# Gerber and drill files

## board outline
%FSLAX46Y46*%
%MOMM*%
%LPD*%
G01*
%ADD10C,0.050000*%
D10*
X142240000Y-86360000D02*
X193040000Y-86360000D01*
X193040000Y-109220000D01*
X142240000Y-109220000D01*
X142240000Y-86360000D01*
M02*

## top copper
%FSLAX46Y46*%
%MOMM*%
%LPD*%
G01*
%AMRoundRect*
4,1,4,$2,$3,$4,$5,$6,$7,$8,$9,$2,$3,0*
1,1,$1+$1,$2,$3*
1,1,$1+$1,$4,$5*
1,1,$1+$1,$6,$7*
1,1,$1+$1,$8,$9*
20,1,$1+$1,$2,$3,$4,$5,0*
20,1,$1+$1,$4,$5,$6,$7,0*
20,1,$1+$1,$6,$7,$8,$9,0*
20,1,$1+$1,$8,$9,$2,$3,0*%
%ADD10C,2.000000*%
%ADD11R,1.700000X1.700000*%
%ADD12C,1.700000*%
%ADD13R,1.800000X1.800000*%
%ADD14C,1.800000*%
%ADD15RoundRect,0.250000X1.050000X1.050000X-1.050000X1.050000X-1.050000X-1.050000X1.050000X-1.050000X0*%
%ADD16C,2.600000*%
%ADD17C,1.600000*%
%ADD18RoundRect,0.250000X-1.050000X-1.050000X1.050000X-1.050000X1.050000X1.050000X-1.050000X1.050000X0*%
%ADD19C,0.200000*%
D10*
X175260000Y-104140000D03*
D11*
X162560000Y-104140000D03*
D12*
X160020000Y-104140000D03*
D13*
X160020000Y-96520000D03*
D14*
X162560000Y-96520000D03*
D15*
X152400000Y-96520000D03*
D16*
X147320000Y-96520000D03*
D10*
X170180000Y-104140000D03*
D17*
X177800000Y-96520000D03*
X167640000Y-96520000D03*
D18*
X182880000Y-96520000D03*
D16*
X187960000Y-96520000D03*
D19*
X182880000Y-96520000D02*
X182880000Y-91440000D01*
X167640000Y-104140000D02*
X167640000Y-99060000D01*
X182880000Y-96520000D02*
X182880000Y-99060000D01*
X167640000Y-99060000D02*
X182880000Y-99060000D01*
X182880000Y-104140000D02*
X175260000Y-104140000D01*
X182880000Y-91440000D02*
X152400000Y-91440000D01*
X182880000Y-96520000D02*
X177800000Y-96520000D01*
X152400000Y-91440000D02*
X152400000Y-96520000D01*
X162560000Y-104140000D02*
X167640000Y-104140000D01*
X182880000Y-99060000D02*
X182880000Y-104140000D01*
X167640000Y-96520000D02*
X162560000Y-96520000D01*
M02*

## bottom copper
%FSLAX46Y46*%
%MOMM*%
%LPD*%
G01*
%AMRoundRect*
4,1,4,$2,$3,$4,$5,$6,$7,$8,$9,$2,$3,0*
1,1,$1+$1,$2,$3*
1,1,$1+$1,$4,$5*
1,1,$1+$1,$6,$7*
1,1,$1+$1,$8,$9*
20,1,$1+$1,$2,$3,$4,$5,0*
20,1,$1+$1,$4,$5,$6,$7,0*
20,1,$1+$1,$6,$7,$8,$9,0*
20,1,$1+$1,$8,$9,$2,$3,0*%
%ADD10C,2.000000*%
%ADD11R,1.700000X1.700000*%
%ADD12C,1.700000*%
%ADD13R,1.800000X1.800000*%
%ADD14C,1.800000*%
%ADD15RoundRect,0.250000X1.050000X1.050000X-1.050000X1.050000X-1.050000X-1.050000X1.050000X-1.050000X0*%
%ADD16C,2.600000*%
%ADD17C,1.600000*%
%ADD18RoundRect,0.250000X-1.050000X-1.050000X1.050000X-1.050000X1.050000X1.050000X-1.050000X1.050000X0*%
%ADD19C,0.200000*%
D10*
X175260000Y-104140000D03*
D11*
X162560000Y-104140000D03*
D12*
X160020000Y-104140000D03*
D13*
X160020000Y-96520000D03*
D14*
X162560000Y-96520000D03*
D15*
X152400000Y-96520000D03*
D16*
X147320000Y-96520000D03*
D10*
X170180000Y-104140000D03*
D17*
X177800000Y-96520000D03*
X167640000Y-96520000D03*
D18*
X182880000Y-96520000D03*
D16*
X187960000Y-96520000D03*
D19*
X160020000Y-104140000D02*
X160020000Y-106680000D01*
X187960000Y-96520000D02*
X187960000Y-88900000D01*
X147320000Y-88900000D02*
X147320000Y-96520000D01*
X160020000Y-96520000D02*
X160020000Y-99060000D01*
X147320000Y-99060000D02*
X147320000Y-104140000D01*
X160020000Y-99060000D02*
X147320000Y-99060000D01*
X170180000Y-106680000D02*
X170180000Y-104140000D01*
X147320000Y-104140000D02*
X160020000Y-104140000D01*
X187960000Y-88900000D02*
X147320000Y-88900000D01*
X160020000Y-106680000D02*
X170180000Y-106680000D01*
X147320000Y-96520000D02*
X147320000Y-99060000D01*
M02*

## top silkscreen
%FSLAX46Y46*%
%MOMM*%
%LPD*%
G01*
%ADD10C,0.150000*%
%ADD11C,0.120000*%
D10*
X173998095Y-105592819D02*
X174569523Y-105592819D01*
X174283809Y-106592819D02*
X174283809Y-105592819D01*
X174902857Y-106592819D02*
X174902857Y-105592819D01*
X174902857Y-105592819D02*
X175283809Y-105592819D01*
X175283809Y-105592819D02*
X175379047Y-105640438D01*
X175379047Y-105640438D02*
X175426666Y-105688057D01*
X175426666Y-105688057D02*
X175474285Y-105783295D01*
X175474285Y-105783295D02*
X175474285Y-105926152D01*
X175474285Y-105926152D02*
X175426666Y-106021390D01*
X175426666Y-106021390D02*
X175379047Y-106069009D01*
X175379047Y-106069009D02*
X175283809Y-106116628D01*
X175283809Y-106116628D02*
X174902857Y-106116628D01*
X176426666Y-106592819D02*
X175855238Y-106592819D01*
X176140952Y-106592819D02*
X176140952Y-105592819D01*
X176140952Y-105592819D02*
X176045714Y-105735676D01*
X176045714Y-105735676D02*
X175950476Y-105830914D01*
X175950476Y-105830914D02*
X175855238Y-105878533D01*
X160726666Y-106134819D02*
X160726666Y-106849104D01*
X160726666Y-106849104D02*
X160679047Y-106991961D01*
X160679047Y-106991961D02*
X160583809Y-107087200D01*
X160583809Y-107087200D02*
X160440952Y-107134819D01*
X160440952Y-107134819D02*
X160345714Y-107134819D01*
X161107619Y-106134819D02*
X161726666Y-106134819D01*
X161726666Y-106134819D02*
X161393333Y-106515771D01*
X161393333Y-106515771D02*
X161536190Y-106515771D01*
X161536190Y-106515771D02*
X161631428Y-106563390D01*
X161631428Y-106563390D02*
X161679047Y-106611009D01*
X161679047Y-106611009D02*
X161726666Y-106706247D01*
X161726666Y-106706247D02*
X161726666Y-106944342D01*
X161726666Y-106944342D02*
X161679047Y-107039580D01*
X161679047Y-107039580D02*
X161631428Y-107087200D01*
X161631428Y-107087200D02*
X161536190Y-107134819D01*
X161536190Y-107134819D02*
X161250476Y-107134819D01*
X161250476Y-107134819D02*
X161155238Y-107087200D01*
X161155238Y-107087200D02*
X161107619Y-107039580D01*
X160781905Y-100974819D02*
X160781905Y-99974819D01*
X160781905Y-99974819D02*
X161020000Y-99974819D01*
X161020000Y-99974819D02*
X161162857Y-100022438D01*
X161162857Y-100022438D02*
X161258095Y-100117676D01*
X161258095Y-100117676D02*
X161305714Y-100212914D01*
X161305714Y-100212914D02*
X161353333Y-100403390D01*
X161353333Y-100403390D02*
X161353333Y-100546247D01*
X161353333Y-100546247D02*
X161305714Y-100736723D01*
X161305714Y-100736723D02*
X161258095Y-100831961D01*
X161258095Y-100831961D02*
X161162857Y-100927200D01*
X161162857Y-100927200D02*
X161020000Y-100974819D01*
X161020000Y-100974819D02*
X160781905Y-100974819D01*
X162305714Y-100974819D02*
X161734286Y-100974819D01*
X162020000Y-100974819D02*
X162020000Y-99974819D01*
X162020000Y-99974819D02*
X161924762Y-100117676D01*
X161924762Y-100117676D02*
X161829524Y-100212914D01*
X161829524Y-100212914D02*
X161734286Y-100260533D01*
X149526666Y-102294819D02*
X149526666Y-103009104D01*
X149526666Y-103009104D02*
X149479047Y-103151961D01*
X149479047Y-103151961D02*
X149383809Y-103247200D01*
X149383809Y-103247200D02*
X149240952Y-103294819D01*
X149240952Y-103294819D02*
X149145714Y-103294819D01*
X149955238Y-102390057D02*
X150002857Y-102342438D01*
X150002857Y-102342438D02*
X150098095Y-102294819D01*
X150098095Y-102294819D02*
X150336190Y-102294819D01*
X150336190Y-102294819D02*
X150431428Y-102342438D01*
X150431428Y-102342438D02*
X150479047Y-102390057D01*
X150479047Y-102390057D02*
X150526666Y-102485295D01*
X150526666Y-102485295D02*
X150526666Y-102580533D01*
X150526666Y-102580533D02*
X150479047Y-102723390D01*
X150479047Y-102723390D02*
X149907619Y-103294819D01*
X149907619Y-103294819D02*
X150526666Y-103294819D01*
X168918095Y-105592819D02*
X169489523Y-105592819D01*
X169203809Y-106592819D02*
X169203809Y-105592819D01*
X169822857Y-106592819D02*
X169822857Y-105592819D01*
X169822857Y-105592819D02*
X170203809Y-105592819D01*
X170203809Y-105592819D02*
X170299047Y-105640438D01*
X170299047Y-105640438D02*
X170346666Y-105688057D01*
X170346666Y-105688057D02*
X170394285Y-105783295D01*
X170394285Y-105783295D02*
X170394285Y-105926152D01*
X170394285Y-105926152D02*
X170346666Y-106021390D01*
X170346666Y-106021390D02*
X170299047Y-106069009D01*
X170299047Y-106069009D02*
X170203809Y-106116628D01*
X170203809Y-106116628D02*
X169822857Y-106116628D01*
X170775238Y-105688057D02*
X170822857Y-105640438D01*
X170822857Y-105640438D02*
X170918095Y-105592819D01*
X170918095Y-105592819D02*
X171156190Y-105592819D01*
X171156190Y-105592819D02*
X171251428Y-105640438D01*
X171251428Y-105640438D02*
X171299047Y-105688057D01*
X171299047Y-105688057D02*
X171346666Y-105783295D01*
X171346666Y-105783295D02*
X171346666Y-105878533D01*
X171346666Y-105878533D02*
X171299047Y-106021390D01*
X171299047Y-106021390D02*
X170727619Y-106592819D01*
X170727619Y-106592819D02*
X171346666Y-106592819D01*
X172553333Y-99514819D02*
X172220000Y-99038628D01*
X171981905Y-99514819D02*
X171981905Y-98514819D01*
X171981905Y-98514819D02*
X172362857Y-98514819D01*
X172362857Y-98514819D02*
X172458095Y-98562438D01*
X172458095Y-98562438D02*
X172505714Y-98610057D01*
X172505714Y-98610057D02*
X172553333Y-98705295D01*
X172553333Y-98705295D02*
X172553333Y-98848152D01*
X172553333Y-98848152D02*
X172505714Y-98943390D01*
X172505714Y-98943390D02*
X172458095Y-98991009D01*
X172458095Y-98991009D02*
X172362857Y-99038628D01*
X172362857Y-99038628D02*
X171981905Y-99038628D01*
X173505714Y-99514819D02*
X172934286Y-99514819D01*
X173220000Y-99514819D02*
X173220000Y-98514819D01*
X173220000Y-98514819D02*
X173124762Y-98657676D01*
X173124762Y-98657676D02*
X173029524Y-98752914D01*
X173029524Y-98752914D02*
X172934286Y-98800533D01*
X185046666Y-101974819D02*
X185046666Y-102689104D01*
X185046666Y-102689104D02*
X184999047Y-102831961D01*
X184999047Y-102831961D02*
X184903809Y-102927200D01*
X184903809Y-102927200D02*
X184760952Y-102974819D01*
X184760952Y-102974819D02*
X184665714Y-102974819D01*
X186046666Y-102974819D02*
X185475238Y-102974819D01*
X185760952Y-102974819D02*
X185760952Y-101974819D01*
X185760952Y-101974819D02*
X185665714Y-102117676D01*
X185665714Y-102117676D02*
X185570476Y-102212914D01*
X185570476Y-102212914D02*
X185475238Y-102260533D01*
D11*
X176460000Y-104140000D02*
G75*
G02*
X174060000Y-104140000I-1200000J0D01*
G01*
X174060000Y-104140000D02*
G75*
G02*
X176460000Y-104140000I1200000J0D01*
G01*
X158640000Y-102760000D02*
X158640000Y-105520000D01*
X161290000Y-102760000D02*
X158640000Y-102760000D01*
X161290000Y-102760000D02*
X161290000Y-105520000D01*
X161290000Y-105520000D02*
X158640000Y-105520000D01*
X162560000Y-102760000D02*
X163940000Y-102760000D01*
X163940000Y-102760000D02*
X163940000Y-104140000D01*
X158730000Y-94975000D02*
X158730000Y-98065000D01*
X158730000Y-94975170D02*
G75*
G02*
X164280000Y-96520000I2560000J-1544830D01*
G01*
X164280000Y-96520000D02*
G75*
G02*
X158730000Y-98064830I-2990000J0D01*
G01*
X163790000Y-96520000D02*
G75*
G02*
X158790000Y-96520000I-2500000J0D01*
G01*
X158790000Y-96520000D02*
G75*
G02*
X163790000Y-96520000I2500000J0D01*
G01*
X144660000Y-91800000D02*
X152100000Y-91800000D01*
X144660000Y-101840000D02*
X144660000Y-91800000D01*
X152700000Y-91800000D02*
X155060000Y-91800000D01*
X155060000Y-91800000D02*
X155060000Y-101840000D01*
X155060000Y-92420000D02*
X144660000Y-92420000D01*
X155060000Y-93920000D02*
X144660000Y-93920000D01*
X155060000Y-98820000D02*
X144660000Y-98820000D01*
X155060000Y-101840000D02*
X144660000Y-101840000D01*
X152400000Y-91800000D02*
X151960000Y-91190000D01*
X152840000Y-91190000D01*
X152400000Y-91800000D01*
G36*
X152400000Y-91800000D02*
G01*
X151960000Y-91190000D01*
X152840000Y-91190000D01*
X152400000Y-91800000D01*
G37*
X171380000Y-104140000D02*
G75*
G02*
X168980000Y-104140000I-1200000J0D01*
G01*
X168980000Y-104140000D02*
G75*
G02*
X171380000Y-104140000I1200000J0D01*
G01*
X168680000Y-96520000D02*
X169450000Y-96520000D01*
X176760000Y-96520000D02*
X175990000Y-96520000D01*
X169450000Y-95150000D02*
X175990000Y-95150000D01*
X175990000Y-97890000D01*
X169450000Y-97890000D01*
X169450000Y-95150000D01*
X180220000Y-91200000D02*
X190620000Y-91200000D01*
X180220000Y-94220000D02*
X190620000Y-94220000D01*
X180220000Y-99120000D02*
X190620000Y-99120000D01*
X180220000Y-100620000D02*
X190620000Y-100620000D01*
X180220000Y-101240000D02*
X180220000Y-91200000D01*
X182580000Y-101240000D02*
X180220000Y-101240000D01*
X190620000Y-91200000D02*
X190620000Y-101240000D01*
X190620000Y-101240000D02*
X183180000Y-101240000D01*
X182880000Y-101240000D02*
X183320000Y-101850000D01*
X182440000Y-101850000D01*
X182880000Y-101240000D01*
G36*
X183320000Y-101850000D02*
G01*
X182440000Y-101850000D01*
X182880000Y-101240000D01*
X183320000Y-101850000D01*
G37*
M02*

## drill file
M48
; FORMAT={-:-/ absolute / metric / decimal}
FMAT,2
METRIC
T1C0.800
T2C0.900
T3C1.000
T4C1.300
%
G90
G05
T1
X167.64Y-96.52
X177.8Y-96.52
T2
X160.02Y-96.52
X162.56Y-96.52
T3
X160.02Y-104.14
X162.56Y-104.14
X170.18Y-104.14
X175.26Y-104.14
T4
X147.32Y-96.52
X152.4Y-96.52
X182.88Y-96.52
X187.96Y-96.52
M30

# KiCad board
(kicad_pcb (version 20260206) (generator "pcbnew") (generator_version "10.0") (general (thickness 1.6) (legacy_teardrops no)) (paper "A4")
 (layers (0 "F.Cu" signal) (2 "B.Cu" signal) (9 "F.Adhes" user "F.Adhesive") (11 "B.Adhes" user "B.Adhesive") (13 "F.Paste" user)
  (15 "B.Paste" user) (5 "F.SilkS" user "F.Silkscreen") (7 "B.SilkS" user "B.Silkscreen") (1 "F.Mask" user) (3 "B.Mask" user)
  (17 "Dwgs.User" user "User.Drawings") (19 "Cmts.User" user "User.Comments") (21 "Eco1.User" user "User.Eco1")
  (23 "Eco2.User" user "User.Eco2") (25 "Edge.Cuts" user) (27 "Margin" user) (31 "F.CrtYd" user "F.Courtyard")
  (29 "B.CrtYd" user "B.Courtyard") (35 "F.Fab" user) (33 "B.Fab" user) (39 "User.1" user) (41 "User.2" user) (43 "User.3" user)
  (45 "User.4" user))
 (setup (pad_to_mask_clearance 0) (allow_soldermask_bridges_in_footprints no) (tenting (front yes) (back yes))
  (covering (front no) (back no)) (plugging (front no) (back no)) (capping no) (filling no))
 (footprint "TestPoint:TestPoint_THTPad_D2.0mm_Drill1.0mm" (layer "F.Cu") (at 175.26 104.14 180)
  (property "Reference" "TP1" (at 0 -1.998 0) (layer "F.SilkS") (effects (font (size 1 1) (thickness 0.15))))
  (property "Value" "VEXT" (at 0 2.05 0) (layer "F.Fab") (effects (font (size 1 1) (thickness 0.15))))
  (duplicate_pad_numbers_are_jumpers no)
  (fp_circle (center 0 0) (end 0 1.2) (stroke (width 0.12) (type solid)) (fill no) (layer "F.SilkS"))
  (pad "1" thru_hole circle (at 0 0 180) (size 2 2) (drill 1) (layers "*.Cu" "*.Mask") (remove_unused_layers no) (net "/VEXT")))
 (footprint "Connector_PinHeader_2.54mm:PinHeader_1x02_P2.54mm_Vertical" (layer "F.Cu") (at 162.56 104.14 -90)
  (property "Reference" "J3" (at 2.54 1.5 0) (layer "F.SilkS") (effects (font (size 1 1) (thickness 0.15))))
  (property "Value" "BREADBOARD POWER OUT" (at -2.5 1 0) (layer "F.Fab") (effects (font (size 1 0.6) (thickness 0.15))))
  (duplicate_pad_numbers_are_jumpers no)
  (fp_line (start -1.38 3.92) (end 1.38 3.92) (stroke (width 0.12) (type solid)) (layer "F.SilkS"))
  (fp_line (start -1.38 1.27) (end -1.38 3.92) (stroke (width 0.12) (type solid)) (layer "F.SilkS"))
  (fp_line (start -1.38 1.27) (end 1.38 1.27) (stroke (width 0.12) (type solid)) (layer "F.SilkS"))
  (fp_line (start 1.38 1.27) (end 1.38 3.92) (stroke (width 0.12) (type solid)) (layer "F.SilkS"))
  (fp_line (start -1.38 0) (end -1.38 -1.38) (stroke (width 0.12) (type solid)) (layer "F.SilkS"))
  (fp_line (start -1.38 -1.38) (end 0 -1.38) (stroke (width 0.12) (type solid)) (layer "F.SilkS"))
  (pad "1" thru_hole rect (at 0 0 270) (size 1.7 1.7) (drill 1) (layers "*.Cu" "*.Mask") (remove_unused_layers no) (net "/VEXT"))
  (pad "2" thru_hole circle (at 0 2.54 270) (size 1.7 1.7) (drill 1) (layers "*.Cu" "*.Mask") (remove_unused_layers no) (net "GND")))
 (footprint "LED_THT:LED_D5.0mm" (layer "F.Cu") (at 160.02 96.52)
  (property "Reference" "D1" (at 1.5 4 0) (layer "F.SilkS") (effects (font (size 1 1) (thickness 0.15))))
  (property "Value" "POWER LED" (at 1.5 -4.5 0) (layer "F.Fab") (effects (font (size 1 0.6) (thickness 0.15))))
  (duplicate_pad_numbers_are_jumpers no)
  (fp_line (start -1.29 -1.545) (end -1.29 1.545) (stroke (width 0.12) (type solid)) (layer "F.SilkS"))
  (fp_arc (start -1.29 -1.54483) (mid 2.071779 -2.880495) (end 4.26 0) (stroke (width 0.12) (type solid)) (layer "F.SilkS"))
  (fp_arc (start 4.26 0) (mid 2.071779 2.880495) (end -1.29 1.54483) (stroke (width 0.12) (type solid)) (layer "F.SilkS"))
  (fp_circle (center 1.27 0) (end 3.77 0) (stroke (width 0.12) (type solid)) (fill no) (layer "F.SilkS"))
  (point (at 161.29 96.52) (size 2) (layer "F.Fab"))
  (pad "1" thru_hole rect (at 0 0) (size 1.8 1.8) (drill 0.9) (layers "*.Cu" "*.Mask") (remove_unused_layers no) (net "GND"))
  (pad "2" thru_hole circle (at 2.54 0) (size 1.8 1.8) (drill 0.9) (layers "*.Cu" "*.Mask") (remove_unused_layers no) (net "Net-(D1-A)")))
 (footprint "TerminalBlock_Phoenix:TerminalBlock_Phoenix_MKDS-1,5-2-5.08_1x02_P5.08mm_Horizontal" (layer "F.Cu") (at 152.4 96.52 180)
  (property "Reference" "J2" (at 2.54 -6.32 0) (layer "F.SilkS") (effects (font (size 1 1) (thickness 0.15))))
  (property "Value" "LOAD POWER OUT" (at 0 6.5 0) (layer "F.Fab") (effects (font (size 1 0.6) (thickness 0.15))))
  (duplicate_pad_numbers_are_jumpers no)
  (fp_line (start 7.74 4.72) (end 0.3 4.72) (stroke (width 0.12) (type solid)) (layer "F.SilkS"))
  (fp_line (start 7.74 -5.32) (end 7.74 4.72) (stroke (width 0.12) (type solid)) (layer "F.SilkS"))
  (fp_line (start -0.3 4.72) (end -2.66 4.72) (stroke (width 0.12) (type solid)) (layer "F.SilkS"))
  (fp_line (start -2.66 4.72) (end -2.66 -5.32) (stroke (width 0.12) (type solid)) (layer "F.SilkS"))
  (fp_line (start -2.66 4.1) (end 7.74 4.1) (stroke (width 0.12) (type solid)) (layer "F.SilkS"))
  (fp_line (start -2.66 2.6) (end 7.74 2.6) (stroke (width 0.12) (type solid)) (layer "F.SilkS"))
  (fp_line (start -2.66 -2.3) (end 7.74 -2.3) (stroke (width 0.12) (type solid)) (layer "F.SilkS"))
  (fp_line (start -2.66 -5.32) (end 7.74 -5.32) (stroke (width 0.12) (type solid)) (layer "F.SilkS"))
  (fp_poly (pts (xy 0 4.72) (xy 0.44 5.33) (xy -0.44 5.33)) (stroke (width 0.12) (type solid)) (fill yes) (layer "F.SilkS"))
  (pad "1" thru_hole roundrect (at 0 0 180) (size 2.6 2.6) (drill 1.3) (layers "*.Cu" "*.Mask") (remove_unused_layers no)
   (roundrect_rratio 0.096154) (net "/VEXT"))
  (pad "2" thru_hole circle (at 5.08 0 180) (size 2.6 2.6) (drill 1.3) (layers "*.Cu" "*.Mask") (remove_unused_layers no) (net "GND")))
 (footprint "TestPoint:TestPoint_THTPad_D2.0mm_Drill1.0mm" (layer "F.Cu") (at 170.18 104.14 180)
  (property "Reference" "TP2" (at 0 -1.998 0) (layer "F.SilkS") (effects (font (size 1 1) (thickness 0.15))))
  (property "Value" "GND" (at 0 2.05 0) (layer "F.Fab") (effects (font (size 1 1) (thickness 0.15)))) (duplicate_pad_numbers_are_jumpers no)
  (fp_circle (center 0 0) (end 0 1.2) (stroke (width 0.12) (type solid)) (fill no) (layer "F.SilkS"))
  (pad "1" thru_hole circle (at 0 0 180) (size 2 2) (drill 1) (layers "*.Cu" "*.Mask") (remove_unused_layers no) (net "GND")))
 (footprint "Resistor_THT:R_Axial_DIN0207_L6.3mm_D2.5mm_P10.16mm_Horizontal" (layer "F.Cu") (at 177.8 96.52 180)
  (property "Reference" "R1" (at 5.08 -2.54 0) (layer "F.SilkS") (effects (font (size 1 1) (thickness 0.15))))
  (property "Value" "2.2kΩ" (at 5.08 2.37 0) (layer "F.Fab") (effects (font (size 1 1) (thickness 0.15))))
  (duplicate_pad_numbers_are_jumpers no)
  (fp_line (start 9.12 0) (end 8.35 0) (stroke (width 0.12) (type solid)) (layer "F.SilkS"))
  (fp_line (start 1.04 0) (end 1.81 0) (stroke (width 0.12) (type solid)) (layer "F.SilkS"))
  (fp_rect (start 1.81 -1.37) (end 8.35 1.37) (stroke (width 0.12) (type solid)) (fill no) (layer "F.SilkS"))
  (pad "1" thru_hole circle (at 0 0 180) (size 1.6 1.6) (drill 0.8) (layers "*.Cu" "*.Mask") (remove_unused_layers no) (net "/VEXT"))
  (pad "2" thru_hole circle (at 10.16 0 180) (size 1.6 1.6) (drill 0.8) (layers "*.Cu" "*.Mask") (remove_unused_layers no)
   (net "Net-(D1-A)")))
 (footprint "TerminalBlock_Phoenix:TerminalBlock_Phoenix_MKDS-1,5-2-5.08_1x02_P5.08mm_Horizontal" (layer "F.Cu") (at 182.88 96.52)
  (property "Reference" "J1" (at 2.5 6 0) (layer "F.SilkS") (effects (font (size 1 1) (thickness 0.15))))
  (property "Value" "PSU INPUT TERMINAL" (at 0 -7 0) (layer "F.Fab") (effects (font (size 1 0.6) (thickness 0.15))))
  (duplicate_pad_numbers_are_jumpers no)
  (fp_line (start -2.66 -5.32) (end 7.74 -5.32) (stroke (width 0.12) (type solid)) (layer "F.SilkS"))
  (fp_line (start -2.66 -2.3) (end 7.74 -2.3) (stroke (width 0.12) (type solid)) (layer "F.SilkS"))
  (fp_line (start -2.66 2.6) (end 7.74 2.6) (stroke (width 0.12) (type solid)) (layer "F.SilkS"))
  (fp_line (start -2.66 4.1) (end 7.74 4.1) (stroke (width 0.12) (type solid)) (layer "F.SilkS"))
  (fp_line (start -2.66 4.72) (end -2.66 -5.32) (stroke (width 0.12) (type solid)) (layer "F.SilkS"))
  (fp_line (start -0.3 4.72) (end -2.66 4.72) (stroke (width 0.12) (type solid)) (layer "F.SilkS"))
  (fp_line (start 7.74 -5.32) (end 7.74 4.72) (stroke (width 0.12) (type solid)) (layer "F.SilkS"))
  (fp_line (start 7.74 4.72) (end 0.3 4.72) (stroke (width 0.12) (type solid)) (layer "F.SilkS"))
  (fp_poly (pts (xy 0 4.72) (xy 0.44 5.33) (xy -0.44 5.33)) (stroke (width 0.12) (type solid)) (fill yes) (layer "F.SilkS"))
  (pad "1" thru_hole roundrect (at 0 0) (size 2.6 2.6) (drill 1.3) (layers "*.Cu" "*.Mask") (remove_unused_layers no)
   (roundrect_rratio 0.096154) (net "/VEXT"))
  (pad "2" thru_hole circle (at 5.08 0) (size 2.6 2.6) (drill 1.3) (layers "*.Cu" "*.Mask") (remove_unused_layers no) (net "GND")))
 (gr_rect (start 142.24 86.36) (end 193.04 109.22) (stroke (width 0.05) (type default)) (fill no) (layer "Edge.Cuts"))
 (segment (start 182.88 96.52) (end 182.88 91.44) (width 0.2) (layer "F.Cu") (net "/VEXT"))
 (segment (start 167.64 104.14) (end 167.64 99.06) (width 0.2) (layer "F.Cu") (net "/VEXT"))
 (segment (start 182.88 96.52) (end 182.88 99.06) (width 0.2) (layer "F.Cu") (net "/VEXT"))
 (segment (start 167.64 99.06) (end 182.88 99.06) (width 0.2) (layer "F.Cu") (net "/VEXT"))
 (segment (start 182.88 104.14) (end 175.26 104.14) (width 0.2) (layer "F.Cu") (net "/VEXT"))
 (segment (start 182.88 91.44) (end 152.4 91.44) (width 0.2) (layer "F.Cu") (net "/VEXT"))
 (segment (start 182.88 96.52) (end 177.8 96.52) (width 0.2) (layer "F.Cu") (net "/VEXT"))
 (segment (start 152.4 91.44) (end 152.4 96.52) (width 0.2) (layer "F.Cu") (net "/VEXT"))
 (segment (start 162.56 104.14) (end 167.64 104.14) (width 0.2) (layer "F.Cu") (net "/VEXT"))
 (segment (start 182.88 99.06) (end 182.88 104.14) (width 0.2) (layer "F.Cu") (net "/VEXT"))
 (segment (start 160.02 104.14) (end 160.02 106.68) (width 0.2) (layer "B.Cu") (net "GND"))
 (segment (start 187.96 96.52) (end 187.96 88.9) (width 0.2) (layer "B.Cu") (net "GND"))
 (segment (start 147.32 88.9) (end 147.32 96.52) (width 0.2) (layer "B.Cu") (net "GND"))
 (segment (start 160.02 96.52) (end 160.02 99.06) (width 0.2) (layer "B.Cu") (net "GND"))
 (segment (start 147.32 99.06) (end 147.32 104.14) (width 0.2) (layer "B.Cu") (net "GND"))
 (segment (start 160.02 99.06) (end 147.32 99.06) (width 0.2) (layer "B.Cu") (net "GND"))
 (segment (start 170.18 106.68) (end 170.18 104.14) (width 0.2) (layer "B.Cu") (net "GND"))
 (segment (start 147.32 104.14) (end 160.02 104.14) (width 0.2) (layer "B.Cu") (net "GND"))
 (segment (start 187.96 88.9) (end 147.32 88.9) (width 0.2) (layer "B.Cu") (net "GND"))
 (segment (start 160.02 106.68) (end 170.18 106.68) (width 0.2) (layer "B.Cu") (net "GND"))
 (segment (start 147.32 96.52) (end 147.32 99.06) (width 0.2) (layer "B.Cu") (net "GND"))
 (segment (start 167.64 96.52) (end 162.56 96.52) (width 0.2) (layer "F.Cu") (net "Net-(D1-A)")))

